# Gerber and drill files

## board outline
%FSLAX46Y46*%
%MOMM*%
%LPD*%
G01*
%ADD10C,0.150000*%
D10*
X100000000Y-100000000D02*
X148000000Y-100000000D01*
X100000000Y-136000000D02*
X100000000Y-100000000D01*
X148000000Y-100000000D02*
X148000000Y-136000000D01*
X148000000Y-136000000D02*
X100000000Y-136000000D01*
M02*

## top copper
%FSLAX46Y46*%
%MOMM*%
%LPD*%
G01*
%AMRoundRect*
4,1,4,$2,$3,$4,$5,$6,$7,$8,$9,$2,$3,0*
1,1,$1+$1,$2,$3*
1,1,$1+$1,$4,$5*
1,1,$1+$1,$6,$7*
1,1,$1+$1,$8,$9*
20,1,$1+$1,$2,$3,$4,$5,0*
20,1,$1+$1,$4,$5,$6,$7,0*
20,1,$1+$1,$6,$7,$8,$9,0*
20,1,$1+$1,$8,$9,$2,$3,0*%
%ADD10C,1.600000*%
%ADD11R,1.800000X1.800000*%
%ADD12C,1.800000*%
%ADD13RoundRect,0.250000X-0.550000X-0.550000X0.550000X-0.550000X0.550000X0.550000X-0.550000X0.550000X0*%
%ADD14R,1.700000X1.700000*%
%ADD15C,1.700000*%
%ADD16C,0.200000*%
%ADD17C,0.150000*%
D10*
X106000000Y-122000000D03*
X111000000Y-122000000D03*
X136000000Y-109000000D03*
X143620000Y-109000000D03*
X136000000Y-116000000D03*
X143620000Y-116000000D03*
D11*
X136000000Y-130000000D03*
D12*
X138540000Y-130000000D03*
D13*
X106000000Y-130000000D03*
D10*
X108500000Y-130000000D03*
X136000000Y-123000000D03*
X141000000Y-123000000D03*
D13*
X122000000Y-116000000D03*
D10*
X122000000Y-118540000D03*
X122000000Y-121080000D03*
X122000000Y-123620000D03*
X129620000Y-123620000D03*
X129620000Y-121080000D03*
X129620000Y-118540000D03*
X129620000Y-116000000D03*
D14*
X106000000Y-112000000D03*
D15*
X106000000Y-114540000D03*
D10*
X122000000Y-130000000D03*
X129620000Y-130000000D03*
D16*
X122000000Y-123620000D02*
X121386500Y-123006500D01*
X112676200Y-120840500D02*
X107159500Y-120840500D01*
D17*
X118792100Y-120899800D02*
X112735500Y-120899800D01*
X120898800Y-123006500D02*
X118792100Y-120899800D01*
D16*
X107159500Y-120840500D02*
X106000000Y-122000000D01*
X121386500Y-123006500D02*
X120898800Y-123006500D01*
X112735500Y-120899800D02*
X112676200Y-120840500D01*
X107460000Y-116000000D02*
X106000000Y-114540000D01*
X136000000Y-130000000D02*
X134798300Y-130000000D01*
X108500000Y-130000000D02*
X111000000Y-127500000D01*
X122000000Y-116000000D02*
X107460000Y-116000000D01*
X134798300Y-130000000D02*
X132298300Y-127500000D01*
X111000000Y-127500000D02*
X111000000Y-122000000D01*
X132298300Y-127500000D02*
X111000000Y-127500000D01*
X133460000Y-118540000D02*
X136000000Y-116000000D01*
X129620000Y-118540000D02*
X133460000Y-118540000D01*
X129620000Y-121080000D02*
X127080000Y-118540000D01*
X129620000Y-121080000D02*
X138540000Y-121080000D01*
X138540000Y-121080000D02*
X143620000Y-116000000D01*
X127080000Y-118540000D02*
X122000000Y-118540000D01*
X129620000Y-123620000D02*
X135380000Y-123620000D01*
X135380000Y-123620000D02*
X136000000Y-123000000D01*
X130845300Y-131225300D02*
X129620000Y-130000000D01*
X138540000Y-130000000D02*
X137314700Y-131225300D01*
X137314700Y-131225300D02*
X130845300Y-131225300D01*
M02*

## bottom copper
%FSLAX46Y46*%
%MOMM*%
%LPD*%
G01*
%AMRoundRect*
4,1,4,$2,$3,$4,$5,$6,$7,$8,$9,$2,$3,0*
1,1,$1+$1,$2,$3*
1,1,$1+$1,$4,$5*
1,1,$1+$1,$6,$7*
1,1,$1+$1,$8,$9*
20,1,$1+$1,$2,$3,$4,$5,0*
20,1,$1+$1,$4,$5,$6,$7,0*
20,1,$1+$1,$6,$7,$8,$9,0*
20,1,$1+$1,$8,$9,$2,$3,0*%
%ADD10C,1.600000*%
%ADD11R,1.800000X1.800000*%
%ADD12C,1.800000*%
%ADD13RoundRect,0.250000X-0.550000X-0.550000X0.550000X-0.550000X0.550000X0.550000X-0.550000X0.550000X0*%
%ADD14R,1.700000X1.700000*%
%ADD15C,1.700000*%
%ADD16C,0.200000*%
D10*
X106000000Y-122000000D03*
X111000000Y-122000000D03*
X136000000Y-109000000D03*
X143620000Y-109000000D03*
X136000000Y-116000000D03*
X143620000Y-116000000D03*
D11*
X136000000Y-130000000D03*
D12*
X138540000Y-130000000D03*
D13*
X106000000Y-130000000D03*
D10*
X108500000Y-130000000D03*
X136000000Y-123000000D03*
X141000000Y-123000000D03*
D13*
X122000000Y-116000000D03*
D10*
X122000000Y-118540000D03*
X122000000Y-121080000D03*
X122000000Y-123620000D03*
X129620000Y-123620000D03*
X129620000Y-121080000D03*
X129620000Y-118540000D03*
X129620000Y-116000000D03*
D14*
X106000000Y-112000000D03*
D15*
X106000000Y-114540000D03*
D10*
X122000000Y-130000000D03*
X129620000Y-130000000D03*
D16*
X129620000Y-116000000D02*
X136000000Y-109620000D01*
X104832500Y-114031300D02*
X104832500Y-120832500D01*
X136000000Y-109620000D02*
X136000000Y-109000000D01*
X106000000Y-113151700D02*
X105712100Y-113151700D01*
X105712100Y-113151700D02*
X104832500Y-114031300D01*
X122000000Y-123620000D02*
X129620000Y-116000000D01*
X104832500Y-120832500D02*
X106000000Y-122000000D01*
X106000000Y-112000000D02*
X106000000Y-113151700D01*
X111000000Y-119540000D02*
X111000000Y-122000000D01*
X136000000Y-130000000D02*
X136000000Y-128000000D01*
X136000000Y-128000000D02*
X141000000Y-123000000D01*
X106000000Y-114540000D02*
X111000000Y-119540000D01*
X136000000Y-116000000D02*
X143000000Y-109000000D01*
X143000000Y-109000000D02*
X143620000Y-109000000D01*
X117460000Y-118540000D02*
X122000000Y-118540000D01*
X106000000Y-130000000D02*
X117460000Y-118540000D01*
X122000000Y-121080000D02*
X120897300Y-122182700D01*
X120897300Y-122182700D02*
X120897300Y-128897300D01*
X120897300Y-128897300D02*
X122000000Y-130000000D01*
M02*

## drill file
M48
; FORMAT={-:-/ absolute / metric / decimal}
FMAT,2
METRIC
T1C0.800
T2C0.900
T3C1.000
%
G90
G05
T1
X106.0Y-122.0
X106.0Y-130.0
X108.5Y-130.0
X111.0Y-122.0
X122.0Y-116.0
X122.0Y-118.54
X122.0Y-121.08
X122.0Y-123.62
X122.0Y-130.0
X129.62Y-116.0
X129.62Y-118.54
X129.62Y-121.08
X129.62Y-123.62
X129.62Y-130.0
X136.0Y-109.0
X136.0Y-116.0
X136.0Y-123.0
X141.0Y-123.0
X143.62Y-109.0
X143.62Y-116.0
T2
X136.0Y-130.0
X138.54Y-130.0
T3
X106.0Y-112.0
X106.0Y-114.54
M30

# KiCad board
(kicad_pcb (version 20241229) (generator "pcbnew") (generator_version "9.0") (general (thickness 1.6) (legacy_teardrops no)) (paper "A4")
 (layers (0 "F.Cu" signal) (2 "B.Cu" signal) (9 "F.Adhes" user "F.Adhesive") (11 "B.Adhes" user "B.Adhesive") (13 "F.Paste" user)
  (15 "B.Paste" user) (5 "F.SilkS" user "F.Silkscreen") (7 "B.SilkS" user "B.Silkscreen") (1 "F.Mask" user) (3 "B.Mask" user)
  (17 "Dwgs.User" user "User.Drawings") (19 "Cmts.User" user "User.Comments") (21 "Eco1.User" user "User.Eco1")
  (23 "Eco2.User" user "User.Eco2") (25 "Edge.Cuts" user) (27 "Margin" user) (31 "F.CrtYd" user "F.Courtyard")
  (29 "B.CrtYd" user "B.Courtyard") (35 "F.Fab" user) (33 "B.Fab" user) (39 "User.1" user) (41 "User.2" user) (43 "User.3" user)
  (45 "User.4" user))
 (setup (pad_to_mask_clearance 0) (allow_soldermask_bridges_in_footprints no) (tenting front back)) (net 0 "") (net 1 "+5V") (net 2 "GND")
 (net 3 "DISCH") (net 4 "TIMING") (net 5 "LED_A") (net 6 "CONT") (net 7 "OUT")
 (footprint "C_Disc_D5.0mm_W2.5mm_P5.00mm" (layer "F.Cu") (at 106 122)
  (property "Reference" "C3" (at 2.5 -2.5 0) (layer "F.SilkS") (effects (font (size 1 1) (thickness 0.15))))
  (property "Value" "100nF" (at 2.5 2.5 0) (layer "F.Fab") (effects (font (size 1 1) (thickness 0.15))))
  (pad "1" thru_hole circle (at 0 0) (size 1.6 1.6) (drill 0.8) (layers "*.Cu" "*.Mask") (remove_unused_layers no) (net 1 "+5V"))
  (pad "2" thru_hole circle (at 5 0) (size 1.6 1.6) (drill 0.8) (layers "*.Cu" "*.Mask") (remove_unused_layers no) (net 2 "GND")))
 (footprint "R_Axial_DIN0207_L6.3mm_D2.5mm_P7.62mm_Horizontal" (layer "F.Cu") (at 136 109)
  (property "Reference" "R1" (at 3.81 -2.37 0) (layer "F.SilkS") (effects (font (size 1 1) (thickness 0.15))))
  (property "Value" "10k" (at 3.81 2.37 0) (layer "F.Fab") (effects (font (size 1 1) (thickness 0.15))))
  (pad "1" thru_hole circle (at 0 0) (size 1.6 1.6) (drill 0.8) (layers "*.Cu" "*.Mask") (remove_unused_layers no) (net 1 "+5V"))
  (pad "2" thru_hole circle (at 7.62 0) (size 1.6 1.6) (drill 0.8) (layers "*.Cu" "*.Mask") (remove_unused_layers no) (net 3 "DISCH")))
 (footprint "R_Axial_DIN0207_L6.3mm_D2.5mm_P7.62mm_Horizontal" (layer "F.Cu") (at 136 116)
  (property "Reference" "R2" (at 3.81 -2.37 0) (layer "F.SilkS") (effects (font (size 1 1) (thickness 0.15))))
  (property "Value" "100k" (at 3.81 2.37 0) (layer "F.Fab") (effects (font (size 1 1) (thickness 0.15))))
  (pad "1" thru_hole circle (at 0 0) (size 1.6 1.6) (drill 0.8) (layers "*.Cu" "*.Mask") (remove_unused_layers no) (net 3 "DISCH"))
  (pad "2" thru_hole circle (at 7.62 0) (size 1.6 1.6) (drill 0.8) (layers "*.Cu" "*.Mask") (remove_unused_layers no) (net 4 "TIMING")))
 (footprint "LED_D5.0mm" (layer "F.Cu") (at 136 130)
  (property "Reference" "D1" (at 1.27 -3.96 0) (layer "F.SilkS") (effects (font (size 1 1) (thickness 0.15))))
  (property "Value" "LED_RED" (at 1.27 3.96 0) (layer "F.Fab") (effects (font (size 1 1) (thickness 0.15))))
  (pad "1" thru_hole rect (at 0 0) (size 1.8 1.8) (drill 0.9) (layers "*.Cu" "*.Mask") (remove_unused_layers no) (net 2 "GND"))
  (pad "2" thru_hole circle (at 2.54 0) (size 1.8 1.8) (drill 0.9) (layers "*.Cu" "*.Mask") (remove_unused_layers no) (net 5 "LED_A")))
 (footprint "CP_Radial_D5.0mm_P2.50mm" (layer "F.Cu") (at 106 130)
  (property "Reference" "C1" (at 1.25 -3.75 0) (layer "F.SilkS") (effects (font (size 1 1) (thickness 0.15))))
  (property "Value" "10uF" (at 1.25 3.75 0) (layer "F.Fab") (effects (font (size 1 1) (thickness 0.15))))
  (pad "1" thru_hole roundrect (at 0 0) (size 1.6 1.6) (drill 0.8) (layers "*.Cu" "*.Mask") (remove_unused_layers no)
   (roundrect_rratio 0.15625) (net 4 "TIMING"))
  (pad "2" thru_hole circle (at 2.5 0) (size 1.6 1.6) (drill 0.8) (layers "*.Cu" "*.Mask") (remove_unused_layers no) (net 2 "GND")))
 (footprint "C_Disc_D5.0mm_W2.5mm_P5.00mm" (layer "F.Cu") (at 136 123)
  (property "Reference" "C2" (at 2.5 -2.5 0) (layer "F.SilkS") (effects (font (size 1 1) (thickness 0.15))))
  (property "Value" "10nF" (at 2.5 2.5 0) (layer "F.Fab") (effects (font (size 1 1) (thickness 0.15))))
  (pad "1" thru_hole circle (at 0 0) (size 1.6 1.6) (drill 0.8) (layers "*.Cu" "*.Mask") (remove_unused_layers no) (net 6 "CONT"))
  (pad "2" thru_hole circle (at 5 0) (size 1.6 1.6) (drill 0.8) (layers "*.Cu" "*.Mask") (remove_unused_layers no) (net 2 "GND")))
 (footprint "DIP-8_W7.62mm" (layer "F.Cu") (at 122 116)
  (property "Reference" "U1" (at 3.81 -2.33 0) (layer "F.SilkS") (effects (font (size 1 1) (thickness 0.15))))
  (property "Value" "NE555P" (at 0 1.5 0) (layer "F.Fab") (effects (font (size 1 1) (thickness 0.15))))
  (pad "1" thru_hole roundrect (at 0 0) (size 1.6 1.6) (drill 0.8) (layers "*.Cu" "*.Mask") (remove_unused_layers no)
   (roundrect_rratio 0.15625) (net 2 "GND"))
  (pad "2" thru_hole circle (at 0 2.54) (size 1.6 1.6) (drill 0.8) (layers "*.Cu" "*.Mask") (remove_unused_layers no) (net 4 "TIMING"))
  (pad "3" thru_hole circle (at 0 5.08) (size 1.6 1.6) (drill 0.8) (layers "*.Cu" "*.Mask") (remove_unused_layers no) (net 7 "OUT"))
  (pad "4" thru_hole circle (at 0 7.62) (size 1.6 1.6) (drill 0.8) (layers "*.Cu" "*.Mask") (remove_unused_layers no) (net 1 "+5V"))
  (pad "5" thru_hole circle (at 7.62 7.62) (size 1.6 1.6) (drill 0.8) (layers "*.Cu" "*.Mask") (remove_unused_layers no) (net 6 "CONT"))
  (pad "6" thru_hole circle (at 7.62 5.08) (size 1.6 1.6) (drill 0.8) (layers "*.Cu" "*.Mask") (remove_unused_layers no) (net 4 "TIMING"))
  (pad "7" thru_hole circle (at 7.62 2.54) (size 1.6 1.6) (drill 0.8) (layers "*.Cu" "*.Mask") (remove_unused_layers no) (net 3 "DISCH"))
  (pad "8" thru_hole circle (at 7.62 0) (size 1.6 1.6) (drill 0.8) (layers "*.Cu" "*.Mask") (remove_unused_layers no) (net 1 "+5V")))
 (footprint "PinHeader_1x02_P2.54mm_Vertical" (layer "F.Cu") (at 106 112)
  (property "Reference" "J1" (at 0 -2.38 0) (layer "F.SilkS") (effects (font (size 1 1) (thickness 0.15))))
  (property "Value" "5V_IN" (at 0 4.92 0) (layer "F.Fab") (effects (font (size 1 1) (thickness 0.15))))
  (pad "1" thru_hole rect (at 0 0) (size 1.7 1.7) (drill 1) (layers "*.Cu" "*.Mask") (remove_unused_layers no) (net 1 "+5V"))
  (pad "2" thru_hole circle (at 0 2.54) (size 1.7 1.7) (drill 1) (layers "*.Cu" "*.Mask") (remove_unused_layers no) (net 2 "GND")))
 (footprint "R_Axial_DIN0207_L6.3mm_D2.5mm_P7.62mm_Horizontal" (layer "F.Cu") (at 122 130)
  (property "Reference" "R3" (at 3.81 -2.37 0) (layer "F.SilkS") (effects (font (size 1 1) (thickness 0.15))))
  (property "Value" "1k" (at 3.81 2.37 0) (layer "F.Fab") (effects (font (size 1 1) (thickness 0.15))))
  (pad "1" thru_hole circle (at 0 0) (size 1.6 1.6) (drill 0.8) (layers "*.Cu" "*.Mask") (remove_unused_layers no) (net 7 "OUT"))
  (pad "2" thru_hole circle (at 7.62 0) (size 1.6 1.6) (drill 0.8) (layers "*.Cu" "*.Mask") (remove_unused_layers no) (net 5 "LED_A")))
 (gr_line (start 100 100) (end 148 100) (stroke (width 0.15) (type default)) (layer "Edge.Cuts"))
 (gr_line (start 100 136) (end 100 100) (stroke (width 0.15) (type default)) (layer "Edge.Cuts"))
 (gr_line (start 148 100) (end 148 136) (stroke (width 0.15) (type default)) (layer "Edge.Cuts"))
 (gr_line (start 148 136) (end 100 136) (stroke (width 0.15) (type default)) (layer "Edge.Cuts"))
 (segment (start 122 123.62) (end 121.3865 123.0065) (width 0.2) (layer "F.Cu") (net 1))
 (segment (start 112.6762 120.8405) (end 107.1595 120.8405) (width 0.2) (layer "F.Cu") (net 1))
 (segment (start 118.7921 120.8998) (end 112.7355 120.8998) (width 0.15) (layer "F.Cu") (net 1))
 (segment (start 120.8988 123.0065) (end 118.7921 120.8998) (width 0.15) (layer "F.Cu") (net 1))
 (segment (start 107.1595 120.8405) (end 106 122) (width 0.2) (layer "F.Cu") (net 1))
 (segment (start 121.3865 123.0065) (end 120.8988 123.0065) (width 0.2) (layer "F.Cu") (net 1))
 (segment (start 112.7355 120.8998) (end 112.6762 120.8405) (width 0.2) (layer "F.Cu") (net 1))
 (segment (start 129.62 116) (end 136 109.62) (width 0.2) (layer "B.Cu") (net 1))
 (segment (start 104.8325 114.0313) (end 104.8325 120.8325) (width 0.2) (layer "B.Cu") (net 1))
 (segment (start 136 109.62) (end 136 109) (width 0.2) (layer "B.Cu") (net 1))
 (segment (start 106 113.1517) (end 105.7121 113.1517) (width 0.2) (layer "B.Cu") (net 1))
 (segment (start 105.7121 113.1517) (end 104.8325 114.0313) (width 0.2) (layer "B.Cu") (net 1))
 (segment (start 122 123.62) (end 129.62 116) (width 0.2) (layer "B.Cu") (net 1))
 (segment (start 104.8325 120.8325) (end 106 122) (width 0.2) (layer "B.Cu") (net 1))
 (segment (start 106 112) (end 106 113.1517) (width 0.2) (layer "B.Cu") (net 1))
 (segment (start 107.46 116) (end 106 114.54) (width 0.2) (layer "F.Cu") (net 2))
 (segment (start 136 130) (end 134.7983 130) (width 0.2) (layer "F.Cu") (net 2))
 (segment (start 108.5 130) (end 111 127.5) (width 0.2) (layer "F.Cu") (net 2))
 (segment (start 122 116) (end 107.46 116) (width 0.2) (layer "F.Cu") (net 2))
 (segment (start 134.7983 130) (end 132.2983 127.5) (width 0.2) (layer "F.Cu") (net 2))
 (segment (start 111 127.5) (end 111 122) (width 0.2) (layer "F.Cu") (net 2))
 (segment (start 132.2983 127.5) (end 111 127.5) (width 0.2) (layer "F.Cu") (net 2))
 (segment (start 111 119.54) (end 111 122) (width 0.2) (layer "B.Cu") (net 2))
 (segment (start 136 130) (end 136 128) (width 0.2) (layer "B.Cu") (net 2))
 (segment (start 136 128) (end 141 123) (width 0.2) (layer "B.Cu") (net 2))
 (segment (start 106 114.54) (end 111 119.54) (width 0.2) (layer "B.Cu") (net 2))
 (segment (start 133.46 118.54) (end 136 116) (width 0.2) (layer "F.Cu") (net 3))
 (segment (start 129.62 118.54) (end 133.46 118.54) (width 0.2) (layer "F.Cu") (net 3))
 (segment (start 136 116) (end 143 109) (width 0.2) (layer "B.Cu") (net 3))
 (segment (start 143 109) (end 143.62 109) (width 0.2) (layer "B.Cu") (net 3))
 (segment (start 129.62 121.08) (end 127.08 118.54) (width 0.2) (layer "F.Cu") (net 4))
 (segment (start 129.62 121.08) (end 138.54 121.08) (width 0.2) (layer "F.Cu") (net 4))
 (segment (start 138.54 121.08) (end 143.62 116) (width 0.2) (layer "F.Cu") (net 4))
 (segment (start 127.08 118.54) (end 122 118.54) (width 0.2) (layer "F.Cu") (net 4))
 (segment (start 117.46 118.54) (end 122 118.54) (width 0.2) (layer "B.Cu") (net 4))
 (segment (start 106 130) (end 117.46 118.54) (width 0.2) (layer "B.Cu") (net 4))
 (segment (start 129.62 123.62) (end 135.38 123.62) (width 0.2) (layer "F.Cu") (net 6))
 (segment (start 135.38 123.62) (end 136 123) (width 0.2) (layer "F.Cu") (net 6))
 (segment (start 122 121.08) (end 120.8973 122.1827) (width 0.2) (layer "B.Cu") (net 7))
 (segment (start 120.8973 122.1827) (end 120.8973 128.8973) (width 0.2) (layer "B.Cu") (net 7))
 (segment (start 120.8973 128.8973) (end 122 130) (width 0.2) (layer "B.Cu") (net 7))
 (segment (start 130.8453 131.2253) (end 129.62 130) (width 0.2) (layer "F.Cu") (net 5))
 (segment (start 138.54 130) (end 137.3147 131.2253) (width 0.2) (layer "F.Cu") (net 5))
 (segment (start 137.3147 131.2253) (end 130.8453 131.2253) (width 0.2) (layer "F.Cu") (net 5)))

